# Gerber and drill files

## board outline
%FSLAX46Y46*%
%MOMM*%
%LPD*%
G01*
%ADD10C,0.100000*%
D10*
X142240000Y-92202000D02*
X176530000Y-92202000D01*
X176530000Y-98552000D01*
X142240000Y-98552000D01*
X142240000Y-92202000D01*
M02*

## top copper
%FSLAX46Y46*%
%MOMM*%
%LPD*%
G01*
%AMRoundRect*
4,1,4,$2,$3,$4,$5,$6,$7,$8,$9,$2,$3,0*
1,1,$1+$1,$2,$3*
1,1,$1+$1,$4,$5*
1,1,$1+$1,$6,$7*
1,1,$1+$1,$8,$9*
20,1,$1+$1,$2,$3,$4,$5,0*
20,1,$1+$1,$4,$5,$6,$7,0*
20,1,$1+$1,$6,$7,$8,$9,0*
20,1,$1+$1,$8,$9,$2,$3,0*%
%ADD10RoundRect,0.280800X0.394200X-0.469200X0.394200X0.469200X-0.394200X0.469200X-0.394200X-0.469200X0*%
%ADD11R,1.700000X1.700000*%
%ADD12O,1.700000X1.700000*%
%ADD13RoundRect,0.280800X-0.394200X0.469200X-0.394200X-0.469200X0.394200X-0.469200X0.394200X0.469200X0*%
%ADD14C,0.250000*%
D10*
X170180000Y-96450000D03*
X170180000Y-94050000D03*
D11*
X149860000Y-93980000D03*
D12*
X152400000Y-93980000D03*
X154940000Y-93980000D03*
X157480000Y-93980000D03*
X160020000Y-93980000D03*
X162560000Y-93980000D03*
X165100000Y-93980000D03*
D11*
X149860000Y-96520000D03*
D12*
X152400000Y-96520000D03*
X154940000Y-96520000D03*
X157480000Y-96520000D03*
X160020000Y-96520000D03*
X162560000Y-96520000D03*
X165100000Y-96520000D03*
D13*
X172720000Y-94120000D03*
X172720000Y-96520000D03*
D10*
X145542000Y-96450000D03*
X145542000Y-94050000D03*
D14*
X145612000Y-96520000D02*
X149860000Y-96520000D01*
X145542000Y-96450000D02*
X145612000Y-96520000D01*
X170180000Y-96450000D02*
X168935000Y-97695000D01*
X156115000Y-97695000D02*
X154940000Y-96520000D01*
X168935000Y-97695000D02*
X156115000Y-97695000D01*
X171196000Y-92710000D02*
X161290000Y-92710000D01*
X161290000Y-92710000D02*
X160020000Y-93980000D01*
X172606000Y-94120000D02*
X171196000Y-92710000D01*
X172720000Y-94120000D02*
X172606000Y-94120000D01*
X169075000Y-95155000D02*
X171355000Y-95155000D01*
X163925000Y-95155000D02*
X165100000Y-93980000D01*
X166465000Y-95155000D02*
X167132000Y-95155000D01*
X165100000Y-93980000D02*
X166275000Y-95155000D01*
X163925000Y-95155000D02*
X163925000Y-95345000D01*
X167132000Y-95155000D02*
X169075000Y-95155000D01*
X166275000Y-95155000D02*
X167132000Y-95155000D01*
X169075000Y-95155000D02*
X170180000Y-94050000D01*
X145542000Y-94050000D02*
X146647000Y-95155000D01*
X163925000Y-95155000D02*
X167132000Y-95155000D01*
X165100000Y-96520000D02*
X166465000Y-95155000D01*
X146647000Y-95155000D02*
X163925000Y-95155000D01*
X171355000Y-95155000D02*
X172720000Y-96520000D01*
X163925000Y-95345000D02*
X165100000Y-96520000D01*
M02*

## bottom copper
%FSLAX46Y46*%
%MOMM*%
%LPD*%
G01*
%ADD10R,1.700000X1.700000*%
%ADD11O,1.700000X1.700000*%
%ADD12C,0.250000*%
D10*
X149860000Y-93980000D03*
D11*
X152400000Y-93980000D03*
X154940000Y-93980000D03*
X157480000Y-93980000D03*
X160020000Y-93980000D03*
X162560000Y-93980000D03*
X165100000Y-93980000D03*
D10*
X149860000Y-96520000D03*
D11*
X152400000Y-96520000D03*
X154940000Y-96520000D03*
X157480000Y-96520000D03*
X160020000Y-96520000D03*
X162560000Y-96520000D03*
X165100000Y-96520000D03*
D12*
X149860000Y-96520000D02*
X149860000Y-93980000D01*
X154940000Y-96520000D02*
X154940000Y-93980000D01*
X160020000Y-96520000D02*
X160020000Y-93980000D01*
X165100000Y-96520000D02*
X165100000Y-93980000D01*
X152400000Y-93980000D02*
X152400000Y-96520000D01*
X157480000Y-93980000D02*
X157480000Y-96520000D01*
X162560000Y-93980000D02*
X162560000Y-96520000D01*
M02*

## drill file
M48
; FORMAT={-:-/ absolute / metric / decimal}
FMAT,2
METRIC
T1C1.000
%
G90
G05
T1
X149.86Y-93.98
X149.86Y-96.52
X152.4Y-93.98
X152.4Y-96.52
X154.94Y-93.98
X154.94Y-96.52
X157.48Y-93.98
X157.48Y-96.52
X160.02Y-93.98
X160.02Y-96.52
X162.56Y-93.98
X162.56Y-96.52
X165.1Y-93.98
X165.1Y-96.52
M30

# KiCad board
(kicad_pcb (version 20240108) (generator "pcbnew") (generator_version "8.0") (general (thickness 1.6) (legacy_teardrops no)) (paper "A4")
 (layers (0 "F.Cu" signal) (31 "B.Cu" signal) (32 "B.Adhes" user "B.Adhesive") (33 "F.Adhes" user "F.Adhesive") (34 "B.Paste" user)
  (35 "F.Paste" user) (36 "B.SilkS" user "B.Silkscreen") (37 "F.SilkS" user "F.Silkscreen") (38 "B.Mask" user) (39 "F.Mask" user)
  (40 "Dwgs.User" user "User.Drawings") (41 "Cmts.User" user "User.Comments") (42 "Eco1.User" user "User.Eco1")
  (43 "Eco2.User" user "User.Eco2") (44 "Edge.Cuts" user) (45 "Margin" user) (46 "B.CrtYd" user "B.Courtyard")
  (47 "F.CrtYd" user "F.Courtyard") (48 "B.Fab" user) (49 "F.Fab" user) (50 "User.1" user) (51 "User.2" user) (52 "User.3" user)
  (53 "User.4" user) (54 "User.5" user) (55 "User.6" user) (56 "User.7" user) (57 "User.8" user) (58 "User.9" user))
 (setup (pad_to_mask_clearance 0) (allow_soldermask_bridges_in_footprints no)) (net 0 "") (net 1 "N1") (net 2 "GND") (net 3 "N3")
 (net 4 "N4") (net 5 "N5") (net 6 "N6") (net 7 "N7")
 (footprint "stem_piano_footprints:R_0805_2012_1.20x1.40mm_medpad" (layer "F.Cu") (at 170.18 95.25 90)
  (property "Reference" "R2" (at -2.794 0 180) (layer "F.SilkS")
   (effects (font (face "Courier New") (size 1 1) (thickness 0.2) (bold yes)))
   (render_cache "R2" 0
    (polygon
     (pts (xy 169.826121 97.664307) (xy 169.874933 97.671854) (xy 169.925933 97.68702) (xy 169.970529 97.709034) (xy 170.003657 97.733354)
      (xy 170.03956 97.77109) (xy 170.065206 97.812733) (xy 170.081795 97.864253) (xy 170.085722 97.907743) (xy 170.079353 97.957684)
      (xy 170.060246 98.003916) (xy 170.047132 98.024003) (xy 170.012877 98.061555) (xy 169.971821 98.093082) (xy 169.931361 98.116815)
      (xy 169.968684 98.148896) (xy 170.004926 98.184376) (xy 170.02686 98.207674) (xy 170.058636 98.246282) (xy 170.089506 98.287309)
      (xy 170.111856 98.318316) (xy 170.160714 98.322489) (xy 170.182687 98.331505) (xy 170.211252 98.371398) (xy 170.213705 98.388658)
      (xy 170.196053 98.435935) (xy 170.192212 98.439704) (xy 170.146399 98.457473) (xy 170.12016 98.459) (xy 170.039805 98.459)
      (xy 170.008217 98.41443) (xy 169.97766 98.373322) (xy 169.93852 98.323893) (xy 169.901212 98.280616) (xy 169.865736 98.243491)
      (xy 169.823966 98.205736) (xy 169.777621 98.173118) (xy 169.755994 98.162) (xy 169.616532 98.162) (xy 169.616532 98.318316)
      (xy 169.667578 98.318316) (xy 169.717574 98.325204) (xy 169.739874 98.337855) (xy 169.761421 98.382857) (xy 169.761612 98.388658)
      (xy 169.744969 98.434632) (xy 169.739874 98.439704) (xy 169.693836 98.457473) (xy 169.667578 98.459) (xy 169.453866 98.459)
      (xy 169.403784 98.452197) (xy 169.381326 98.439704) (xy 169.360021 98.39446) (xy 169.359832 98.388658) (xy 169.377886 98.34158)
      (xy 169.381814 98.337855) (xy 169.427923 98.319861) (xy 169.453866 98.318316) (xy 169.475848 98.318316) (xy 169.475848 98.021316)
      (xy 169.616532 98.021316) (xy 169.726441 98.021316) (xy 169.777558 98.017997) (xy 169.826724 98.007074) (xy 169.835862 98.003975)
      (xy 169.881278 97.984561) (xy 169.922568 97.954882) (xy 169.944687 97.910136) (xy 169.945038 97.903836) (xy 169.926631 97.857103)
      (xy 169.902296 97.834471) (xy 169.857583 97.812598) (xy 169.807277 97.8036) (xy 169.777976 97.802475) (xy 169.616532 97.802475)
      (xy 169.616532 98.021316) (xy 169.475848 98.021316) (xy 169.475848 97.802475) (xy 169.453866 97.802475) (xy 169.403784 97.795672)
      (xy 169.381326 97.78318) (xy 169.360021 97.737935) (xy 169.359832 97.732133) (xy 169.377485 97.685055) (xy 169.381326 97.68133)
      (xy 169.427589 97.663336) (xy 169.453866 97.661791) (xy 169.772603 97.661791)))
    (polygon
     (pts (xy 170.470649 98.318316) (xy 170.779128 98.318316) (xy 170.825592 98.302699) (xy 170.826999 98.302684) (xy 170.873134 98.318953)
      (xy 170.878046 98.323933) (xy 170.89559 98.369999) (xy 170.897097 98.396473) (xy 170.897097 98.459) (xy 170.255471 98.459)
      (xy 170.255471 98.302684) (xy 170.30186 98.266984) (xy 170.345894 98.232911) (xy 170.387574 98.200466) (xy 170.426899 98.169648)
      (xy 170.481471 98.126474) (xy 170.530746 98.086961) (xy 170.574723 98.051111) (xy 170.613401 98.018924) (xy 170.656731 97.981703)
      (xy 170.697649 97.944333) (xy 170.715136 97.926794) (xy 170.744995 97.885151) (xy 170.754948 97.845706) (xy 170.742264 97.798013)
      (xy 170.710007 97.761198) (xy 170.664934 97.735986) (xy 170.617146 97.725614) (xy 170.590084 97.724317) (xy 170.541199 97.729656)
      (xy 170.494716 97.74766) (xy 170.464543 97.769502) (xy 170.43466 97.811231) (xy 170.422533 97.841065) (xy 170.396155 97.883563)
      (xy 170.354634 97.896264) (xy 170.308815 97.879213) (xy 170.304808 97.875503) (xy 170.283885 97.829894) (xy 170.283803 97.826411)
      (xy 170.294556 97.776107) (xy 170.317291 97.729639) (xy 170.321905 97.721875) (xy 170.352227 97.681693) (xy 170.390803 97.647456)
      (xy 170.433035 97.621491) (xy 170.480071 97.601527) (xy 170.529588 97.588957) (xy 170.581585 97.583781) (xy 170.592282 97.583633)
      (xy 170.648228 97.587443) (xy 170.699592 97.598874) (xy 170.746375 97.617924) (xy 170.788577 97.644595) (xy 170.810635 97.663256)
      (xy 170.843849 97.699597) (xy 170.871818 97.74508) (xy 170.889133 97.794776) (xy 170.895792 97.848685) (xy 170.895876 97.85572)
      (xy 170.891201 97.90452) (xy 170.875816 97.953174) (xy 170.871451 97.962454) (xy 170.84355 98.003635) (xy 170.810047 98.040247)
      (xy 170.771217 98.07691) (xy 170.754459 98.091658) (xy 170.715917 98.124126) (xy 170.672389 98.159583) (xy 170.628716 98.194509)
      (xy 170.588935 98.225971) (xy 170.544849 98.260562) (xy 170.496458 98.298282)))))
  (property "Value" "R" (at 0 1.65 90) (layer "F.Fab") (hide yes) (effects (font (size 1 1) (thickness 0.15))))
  (pad "1" smd roundrect (at -1.2 0 90) (size 1.5 1.35) (layers "F.Cu" "F.Paste" "F.Mask") (roundrect_rratio 0.208) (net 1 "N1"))
  (pad "2" smd roundrect (at 1.2 0 90) (size 1.5 1.35) (layers "F.Cu" "F.Paste" "F.Mask") (roundrect_rratio 0.208) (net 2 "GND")))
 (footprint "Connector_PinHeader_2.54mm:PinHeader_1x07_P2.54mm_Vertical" (layer "F.Cu") (at 149.86 93.98 90)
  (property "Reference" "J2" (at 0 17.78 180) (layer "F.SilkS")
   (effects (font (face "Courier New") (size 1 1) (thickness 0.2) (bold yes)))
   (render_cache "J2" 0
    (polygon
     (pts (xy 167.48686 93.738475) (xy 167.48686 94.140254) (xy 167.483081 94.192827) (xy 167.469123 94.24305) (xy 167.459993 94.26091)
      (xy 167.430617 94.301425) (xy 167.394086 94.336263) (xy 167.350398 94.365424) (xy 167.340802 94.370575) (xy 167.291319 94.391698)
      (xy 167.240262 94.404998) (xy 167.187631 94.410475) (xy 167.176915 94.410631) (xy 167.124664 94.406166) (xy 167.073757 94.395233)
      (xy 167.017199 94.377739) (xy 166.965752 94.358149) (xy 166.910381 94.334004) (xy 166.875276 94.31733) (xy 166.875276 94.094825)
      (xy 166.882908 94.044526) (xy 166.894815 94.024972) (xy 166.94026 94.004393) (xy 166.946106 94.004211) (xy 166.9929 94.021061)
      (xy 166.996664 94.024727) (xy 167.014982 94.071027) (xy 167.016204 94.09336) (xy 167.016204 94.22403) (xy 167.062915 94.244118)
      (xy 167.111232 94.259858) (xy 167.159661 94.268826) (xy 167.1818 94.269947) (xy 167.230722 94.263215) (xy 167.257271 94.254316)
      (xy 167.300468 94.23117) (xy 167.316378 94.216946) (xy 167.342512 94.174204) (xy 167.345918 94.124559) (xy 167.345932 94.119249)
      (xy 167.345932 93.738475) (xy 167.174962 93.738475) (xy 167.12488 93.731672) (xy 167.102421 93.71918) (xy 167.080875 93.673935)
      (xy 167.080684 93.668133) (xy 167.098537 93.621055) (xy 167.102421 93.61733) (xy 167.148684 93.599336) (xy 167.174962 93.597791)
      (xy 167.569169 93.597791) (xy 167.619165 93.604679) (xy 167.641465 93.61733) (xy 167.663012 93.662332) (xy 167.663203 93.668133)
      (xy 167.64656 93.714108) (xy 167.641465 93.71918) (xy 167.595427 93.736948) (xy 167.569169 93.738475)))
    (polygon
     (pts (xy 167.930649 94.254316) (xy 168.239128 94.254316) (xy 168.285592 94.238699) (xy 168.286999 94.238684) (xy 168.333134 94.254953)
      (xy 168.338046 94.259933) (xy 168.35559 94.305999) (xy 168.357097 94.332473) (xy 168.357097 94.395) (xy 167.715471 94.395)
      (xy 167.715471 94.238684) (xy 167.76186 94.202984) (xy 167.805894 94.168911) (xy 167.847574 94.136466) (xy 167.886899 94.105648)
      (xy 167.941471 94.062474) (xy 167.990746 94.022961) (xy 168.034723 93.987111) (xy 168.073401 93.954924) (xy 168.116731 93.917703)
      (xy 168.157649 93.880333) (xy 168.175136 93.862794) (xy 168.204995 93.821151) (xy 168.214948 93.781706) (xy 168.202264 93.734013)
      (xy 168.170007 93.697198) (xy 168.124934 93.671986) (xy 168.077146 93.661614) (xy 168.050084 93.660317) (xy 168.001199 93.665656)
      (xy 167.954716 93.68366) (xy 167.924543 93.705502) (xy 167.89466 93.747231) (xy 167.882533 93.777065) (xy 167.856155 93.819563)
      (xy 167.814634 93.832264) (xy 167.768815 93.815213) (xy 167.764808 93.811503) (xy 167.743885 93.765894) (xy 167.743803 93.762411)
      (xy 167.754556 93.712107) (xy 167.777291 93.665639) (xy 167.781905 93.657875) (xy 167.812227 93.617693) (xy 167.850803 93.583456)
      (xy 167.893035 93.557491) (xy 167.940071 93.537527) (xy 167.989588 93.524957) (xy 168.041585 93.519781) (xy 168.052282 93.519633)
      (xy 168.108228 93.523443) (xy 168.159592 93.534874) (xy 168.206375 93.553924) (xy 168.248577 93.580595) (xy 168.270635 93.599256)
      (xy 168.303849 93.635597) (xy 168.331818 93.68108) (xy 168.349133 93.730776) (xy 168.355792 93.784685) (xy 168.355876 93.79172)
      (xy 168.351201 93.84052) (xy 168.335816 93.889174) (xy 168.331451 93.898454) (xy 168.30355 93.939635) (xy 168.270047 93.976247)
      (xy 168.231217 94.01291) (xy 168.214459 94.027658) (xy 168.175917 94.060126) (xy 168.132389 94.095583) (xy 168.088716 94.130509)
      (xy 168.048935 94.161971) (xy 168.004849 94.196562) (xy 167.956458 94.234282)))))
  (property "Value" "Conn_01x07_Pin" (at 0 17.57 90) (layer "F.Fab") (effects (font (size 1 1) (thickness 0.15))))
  (pad "1" thru_hole rect (at 0 0 90) (size 1.7 1.7) (drill 1) (layers "*.Cu" "*.Mask") (remove_unused_layers no) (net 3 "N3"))
  (pad "2" thru_hole oval (at 0 2.54 90) (size 1.7 1.7) (drill 1) (layers "*.Cu" "*.Mask") (remove_unused_layers no) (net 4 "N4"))
  (pad "3" thru_hole oval (at 0 5.08 90) (size 1.7 1.7) (drill 1) (layers "*.Cu" "*.Mask") (remove_unused_layers no) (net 1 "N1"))
  (pad "4" thru_hole oval (at 0 7.62 90) (size 1.7 1.7) (drill 1) (layers "*.Cu" "*.Mask") (remove_unused_layers no) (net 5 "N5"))
  (pad "5" thru_hole oval (at 0 10.16 90) (size 1.7 1.7) (drill 1) (layers "*.Cu" "*.Mask") (remove_unused_layers no) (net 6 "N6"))
  (pad "6" thru_hole oval (at 0 12.7 90) (size 1.7 1.7) (drill 1) (layers "*.Cu" "*.Mask") (remove_unused_layers no) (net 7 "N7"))
  (pad "7" thru_hole oval (at 0 15.24 90) (size 1.7 1.7) (drill 1) (layers "*.Cu" "*.Mask") (remove_unused_layers no) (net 2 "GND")))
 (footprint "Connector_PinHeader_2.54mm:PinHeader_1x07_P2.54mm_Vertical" (layer "F.Cu") (at 149.86 96.52 90)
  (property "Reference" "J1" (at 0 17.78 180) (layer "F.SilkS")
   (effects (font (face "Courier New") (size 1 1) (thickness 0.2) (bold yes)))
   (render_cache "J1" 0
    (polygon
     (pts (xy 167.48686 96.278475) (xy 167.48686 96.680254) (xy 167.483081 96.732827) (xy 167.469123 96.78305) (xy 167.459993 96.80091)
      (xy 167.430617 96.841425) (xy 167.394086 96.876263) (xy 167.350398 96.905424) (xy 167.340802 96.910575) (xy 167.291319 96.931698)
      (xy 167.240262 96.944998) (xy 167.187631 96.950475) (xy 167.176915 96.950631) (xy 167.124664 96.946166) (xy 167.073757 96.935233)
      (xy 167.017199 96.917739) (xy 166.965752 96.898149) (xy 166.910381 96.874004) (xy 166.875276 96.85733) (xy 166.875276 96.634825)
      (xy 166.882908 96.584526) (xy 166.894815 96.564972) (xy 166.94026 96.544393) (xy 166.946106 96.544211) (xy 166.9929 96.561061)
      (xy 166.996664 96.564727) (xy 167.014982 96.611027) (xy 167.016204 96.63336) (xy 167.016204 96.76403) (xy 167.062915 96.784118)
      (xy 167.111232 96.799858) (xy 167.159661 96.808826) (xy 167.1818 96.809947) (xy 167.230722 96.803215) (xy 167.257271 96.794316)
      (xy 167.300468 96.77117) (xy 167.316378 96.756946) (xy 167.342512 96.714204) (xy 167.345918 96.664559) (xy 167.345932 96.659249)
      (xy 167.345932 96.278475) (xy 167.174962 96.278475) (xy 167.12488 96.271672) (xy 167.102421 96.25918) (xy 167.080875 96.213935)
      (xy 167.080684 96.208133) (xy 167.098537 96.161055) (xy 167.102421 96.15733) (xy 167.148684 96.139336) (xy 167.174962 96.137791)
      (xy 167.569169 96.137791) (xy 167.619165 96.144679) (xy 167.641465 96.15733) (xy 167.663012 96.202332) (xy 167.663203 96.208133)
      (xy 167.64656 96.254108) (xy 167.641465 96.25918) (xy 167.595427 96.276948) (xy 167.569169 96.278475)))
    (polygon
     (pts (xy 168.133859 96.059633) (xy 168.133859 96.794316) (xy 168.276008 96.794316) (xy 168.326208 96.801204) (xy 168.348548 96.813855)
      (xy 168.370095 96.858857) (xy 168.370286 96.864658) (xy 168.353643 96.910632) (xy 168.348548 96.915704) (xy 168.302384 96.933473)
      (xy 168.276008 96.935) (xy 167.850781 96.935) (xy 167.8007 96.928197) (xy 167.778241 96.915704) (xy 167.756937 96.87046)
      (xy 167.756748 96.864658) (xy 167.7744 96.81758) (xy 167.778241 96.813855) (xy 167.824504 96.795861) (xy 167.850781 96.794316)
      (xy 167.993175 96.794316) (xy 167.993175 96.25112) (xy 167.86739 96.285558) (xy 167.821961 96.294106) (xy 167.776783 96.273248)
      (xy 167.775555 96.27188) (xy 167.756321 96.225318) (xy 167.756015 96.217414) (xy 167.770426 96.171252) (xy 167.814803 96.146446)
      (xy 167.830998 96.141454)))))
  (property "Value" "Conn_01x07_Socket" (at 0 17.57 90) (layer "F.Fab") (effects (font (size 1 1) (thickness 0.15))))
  (pad "1" thru_hole rect (at 0 0 90) (size 1.7 1.7) (drill 1) (layers "*.Cu" "*.Mask") (remove_unused_layers no) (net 3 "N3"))
  (pad "2" thru_hole oval (at 0 2.54 90) (size 1.7 1.7) (drill 1) (layers "*.Cu" "*.Mask") (remove_unused_layers no) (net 4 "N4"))
  (pad "3" thru_hole oval (at 0 5.08 90) (size 1.7 1.7) (drill 1) (layers "*.Cu" "*.Mask") (remove_unused_layers no) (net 1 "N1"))
  (pad "4" thru_hole oval (at 0 7.62 90) (size 1.7 1.7) (drill 1) (layers "*.Cu" "*.Mask") (remove_unused_layers no) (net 5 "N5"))
  (pad "5" thru_hole oval (at 0 10.16 90) (size 1.7 1.7) (drill 1) (layers "*.Cu" "*.Mask") (remove_unused_layers no) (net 6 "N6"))
  (pad "6" thru_hole oval (at 0 12.7 90) (size 1.7 1.7) (drill 1) (layers "*.Cu" "*.Mask") (remove_unused_layers no) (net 7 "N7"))
  (pad "7" thru_hole oval (at 0 15.24 90) (size 1.7 1.7) (drill 1) (layers "*.Cu" "*.Mask") (remove_unused_layers no) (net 2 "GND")))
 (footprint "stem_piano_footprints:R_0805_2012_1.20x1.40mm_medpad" (layer "F.Cu") (at 172.72 95.32 -90)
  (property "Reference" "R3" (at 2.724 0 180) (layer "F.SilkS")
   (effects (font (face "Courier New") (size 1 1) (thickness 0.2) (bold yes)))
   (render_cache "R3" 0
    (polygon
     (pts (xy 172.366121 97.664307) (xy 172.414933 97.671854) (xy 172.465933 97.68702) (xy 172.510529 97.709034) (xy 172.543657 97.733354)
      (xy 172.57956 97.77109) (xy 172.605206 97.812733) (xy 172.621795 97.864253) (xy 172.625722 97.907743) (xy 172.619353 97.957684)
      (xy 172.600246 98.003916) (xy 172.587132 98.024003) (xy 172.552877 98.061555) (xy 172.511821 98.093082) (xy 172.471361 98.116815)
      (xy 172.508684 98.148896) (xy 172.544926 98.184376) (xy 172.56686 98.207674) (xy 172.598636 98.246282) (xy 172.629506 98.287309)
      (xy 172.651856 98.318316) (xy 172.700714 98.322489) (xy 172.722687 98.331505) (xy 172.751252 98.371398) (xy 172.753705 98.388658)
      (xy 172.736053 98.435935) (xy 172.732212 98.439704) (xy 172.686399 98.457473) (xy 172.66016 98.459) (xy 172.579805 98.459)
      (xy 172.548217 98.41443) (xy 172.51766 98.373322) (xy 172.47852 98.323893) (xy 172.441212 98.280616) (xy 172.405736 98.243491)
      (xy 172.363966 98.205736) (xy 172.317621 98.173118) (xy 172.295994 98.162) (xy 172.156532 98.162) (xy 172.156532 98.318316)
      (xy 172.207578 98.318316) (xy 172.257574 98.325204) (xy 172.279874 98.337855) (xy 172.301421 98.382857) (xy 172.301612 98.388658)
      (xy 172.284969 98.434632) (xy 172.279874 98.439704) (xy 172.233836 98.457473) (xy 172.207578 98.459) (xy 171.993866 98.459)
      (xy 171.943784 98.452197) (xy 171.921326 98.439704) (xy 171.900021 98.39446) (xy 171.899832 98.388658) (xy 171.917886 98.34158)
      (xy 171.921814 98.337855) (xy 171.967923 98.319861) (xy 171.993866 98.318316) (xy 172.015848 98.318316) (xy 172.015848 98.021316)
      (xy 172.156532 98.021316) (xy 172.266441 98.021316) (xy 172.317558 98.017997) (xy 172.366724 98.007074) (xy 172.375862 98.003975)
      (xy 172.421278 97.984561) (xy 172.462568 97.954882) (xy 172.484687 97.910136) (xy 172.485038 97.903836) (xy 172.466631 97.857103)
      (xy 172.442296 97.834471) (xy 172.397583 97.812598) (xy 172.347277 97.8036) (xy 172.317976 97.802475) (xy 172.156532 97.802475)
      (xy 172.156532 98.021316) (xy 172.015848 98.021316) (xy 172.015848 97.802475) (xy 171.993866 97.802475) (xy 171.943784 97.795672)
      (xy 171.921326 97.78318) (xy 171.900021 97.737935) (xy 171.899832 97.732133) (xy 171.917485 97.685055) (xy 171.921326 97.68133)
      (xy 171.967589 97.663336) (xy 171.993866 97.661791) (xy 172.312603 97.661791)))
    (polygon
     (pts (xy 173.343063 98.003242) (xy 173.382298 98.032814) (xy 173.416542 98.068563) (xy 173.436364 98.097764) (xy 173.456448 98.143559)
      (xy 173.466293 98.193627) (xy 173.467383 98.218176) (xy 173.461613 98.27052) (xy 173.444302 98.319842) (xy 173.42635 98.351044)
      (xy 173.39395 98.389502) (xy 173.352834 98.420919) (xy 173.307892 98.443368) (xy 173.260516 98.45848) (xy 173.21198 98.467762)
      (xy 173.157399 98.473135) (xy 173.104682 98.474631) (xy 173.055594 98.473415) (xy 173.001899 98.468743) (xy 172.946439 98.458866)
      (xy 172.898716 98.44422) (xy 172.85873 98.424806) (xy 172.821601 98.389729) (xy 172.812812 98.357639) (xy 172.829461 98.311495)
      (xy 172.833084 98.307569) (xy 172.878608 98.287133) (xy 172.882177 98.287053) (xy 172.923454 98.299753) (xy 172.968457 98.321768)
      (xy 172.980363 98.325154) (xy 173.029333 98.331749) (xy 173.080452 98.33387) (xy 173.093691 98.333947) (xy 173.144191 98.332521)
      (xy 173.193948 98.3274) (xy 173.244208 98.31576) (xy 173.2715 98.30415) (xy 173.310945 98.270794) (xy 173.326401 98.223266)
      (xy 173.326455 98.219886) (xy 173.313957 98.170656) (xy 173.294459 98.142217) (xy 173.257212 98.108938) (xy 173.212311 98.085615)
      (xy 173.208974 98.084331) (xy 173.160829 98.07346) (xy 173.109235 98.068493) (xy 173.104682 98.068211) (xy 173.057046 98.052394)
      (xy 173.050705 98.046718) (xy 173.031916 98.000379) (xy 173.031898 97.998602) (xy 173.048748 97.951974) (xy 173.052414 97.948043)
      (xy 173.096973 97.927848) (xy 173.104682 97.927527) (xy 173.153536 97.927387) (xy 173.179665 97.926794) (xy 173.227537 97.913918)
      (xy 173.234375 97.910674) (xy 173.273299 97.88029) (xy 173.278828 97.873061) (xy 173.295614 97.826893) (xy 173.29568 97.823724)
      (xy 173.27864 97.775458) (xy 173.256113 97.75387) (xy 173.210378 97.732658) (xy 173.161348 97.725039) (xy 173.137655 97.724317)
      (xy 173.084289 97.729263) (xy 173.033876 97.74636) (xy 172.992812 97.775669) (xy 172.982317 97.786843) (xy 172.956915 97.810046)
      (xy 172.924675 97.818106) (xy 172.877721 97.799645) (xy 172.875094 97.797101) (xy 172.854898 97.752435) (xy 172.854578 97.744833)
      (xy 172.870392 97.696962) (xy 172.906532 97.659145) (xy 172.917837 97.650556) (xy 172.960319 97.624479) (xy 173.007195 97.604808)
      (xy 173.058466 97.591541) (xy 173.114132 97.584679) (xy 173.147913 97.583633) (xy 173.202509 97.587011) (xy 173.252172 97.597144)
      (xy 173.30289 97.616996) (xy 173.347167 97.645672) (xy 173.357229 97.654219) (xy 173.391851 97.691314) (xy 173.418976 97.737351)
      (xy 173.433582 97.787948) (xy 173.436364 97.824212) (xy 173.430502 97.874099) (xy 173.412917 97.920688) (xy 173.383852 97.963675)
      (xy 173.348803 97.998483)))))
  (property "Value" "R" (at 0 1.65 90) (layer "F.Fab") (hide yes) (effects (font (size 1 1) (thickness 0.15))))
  (pad "1" smd roundrect (at -1.2 0 270) (size 1.5 1.35) (layers "F.Cu" "F.Paste" "F.Mask") (roundrect_rratio 0.208) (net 6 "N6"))
  (pad "2" smd roundrect (at 1.2 0 270) (size 1.5 1.35) (layers "F.Cu" "F.Paste" "F.Mask") (roundrect_rratio 0.208) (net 2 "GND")))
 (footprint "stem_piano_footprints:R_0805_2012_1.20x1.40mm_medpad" (layer "F.Cu") (at 145.542 95.25 90)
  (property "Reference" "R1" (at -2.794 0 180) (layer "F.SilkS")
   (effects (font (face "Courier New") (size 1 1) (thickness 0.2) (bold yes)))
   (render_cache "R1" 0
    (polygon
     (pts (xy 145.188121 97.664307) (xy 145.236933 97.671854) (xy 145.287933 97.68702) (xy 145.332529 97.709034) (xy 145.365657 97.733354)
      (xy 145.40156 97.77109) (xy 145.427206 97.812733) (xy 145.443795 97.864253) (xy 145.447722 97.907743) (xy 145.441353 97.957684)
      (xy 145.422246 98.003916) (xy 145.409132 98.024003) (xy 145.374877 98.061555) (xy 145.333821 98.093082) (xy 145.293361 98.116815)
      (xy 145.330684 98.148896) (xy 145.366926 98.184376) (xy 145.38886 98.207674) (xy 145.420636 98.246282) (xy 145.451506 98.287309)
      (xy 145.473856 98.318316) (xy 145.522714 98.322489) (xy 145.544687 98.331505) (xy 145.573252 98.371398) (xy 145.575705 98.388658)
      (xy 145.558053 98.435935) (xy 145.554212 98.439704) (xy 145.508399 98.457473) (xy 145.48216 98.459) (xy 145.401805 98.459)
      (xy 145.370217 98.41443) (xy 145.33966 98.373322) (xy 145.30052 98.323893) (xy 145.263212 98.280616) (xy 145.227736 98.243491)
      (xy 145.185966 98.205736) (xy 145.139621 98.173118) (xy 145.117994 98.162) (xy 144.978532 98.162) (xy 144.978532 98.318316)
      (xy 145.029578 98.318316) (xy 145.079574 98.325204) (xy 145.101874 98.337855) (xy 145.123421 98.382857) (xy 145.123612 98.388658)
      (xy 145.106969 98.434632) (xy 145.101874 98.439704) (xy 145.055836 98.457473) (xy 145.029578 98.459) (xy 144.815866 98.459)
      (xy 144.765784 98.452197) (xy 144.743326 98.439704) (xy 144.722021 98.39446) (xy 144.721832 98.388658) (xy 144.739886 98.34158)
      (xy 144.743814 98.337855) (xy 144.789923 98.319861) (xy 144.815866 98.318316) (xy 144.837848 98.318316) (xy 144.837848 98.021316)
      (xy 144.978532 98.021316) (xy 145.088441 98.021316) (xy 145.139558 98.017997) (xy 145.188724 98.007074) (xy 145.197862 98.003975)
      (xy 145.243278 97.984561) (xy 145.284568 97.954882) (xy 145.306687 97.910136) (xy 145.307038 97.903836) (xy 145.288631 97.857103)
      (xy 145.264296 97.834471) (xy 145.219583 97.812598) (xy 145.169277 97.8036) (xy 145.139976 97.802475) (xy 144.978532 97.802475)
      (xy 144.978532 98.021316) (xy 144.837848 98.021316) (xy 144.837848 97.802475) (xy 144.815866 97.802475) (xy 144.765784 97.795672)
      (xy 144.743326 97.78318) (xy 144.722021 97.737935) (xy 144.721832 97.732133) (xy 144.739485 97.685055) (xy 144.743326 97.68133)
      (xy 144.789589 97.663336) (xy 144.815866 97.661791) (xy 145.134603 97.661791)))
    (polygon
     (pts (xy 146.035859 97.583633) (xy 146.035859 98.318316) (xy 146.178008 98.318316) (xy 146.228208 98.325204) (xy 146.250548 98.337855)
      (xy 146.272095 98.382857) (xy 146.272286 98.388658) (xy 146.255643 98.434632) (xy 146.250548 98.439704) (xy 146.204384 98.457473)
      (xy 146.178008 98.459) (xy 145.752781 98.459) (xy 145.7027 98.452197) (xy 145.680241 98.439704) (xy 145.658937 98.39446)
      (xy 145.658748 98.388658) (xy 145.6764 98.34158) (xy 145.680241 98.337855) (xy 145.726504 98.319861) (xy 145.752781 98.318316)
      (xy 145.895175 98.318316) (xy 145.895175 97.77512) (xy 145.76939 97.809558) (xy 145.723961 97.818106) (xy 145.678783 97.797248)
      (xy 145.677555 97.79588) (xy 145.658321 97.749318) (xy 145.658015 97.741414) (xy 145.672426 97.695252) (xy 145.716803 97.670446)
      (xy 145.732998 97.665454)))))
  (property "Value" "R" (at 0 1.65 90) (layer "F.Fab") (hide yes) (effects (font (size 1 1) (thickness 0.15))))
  (pad "1" smd roundrect (at -1.2 0 90) (size 1.5 1.35) (layers "F.Cu" "F.Paste" "F.Mask") (roundrect_rratio 0.208) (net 3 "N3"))
  (pad "2" smd roundrect (at 1.2 0 90) (size 1.5 1.35) (layers "F.Cu" "F.Paste" "F.Mask") (roundrect_rratio 0.208) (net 2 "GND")))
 (gr_rect (start 142.24 92.202) (end 176.53 98.552) (stroke (width 0.1) (type default)) (fill none) (layer "Edge.Cuts"))
 (segment (start 145.612 96.52) (end 149.86 96.52) (width 0.25) (layer "F.Cu") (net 3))
 (segment (start 145.542 96.45) (end 145.612 96.52) (width 0.25) (layer "F.Cu") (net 3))
 (segment (start 149.86 96.52) (end 149.86 93.98) (width 0.25) (layer "B.Cu") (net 3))
 (segment (start 170.18 96.45) (end 168.935 97.695) (width 0.25) (layer "F.Cu") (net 1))
 (segment (start 156.115 97.695) (end 154.94 96.52) (width 0.25) (layer "F.Cu") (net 1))
 (segment (start 168.935 97.695) (end 156.115 97.695) (width 0.25) (layer "F.Cu") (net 1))
 (segment (start 154.94 96.52) (end 154.94 93.98) (width 0.25) (layer "B.Cu") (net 1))
 (segment (start 171.196 92.71) (end 161.29 92.71) (width 0.25) (layer "F.Cu") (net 6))
 (segment (start 161.29 92.71) (end 160.02 93.98) (width 0.25) (layer "F.Cu") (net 6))
 (segment (start 172.606 94.12) (end 171.196 92.71) (width 0.25) (layer "F.Cu") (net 6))
 (segment (start 172.72 94.12) (end 172.606 94.12) (width 0.25) (layer "F.Cu") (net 6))
 (segment (start 160.02 96.52) (end 160.02 93.98) (width 0.25) (layer "B.Cu") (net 6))
 (segment (start 169.075 95.155) (end 171.355 95.155) (width 0.25) (layer "F.Cu") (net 2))
 (segment (start 163.925 95.155) (end 165.1 93.98) (width 0.25) (layer "F.Cu") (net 2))
 (segment (start 166.465 95.155) (end 167.132 95.155) (width 0.25) (layer "F.Cu") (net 2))
 (segment (start 165.1 93.98) (end 166.275 95.155) (width 0.25) (layer "F.Cu") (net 2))
 (segment (start 163.925 95.155) (end 163.925 95.345) (width 0.25) (layer "F.Cu") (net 2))
 (segment (start 167.132 95.155) (end 169.075 95.155) (width 0.25) (layer "F.Cu") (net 2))
 (segment (start 166.275 95.155) (end 167.132 95.155) (width 0.25) (layer "F.Cu") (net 2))
 (segment (start 169.075 95.155) (end 170.18 94.05) (width 0.25) (layer "F.Cu") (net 2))
 (segment (start 145.542 94.05) (end 146.647 95.155) (width 0.25) (layer "F.Cu") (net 2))
 (segment (start 163.925 95.155) (end 167.132 95.155) (width 0.25) (layer "F.Cu") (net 2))
 (segment (start 165.1 96.52) (end 166.465 95.155) (width 0.25) (layer "F.Cu") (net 2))
 (segment (start 146.647 95.155) (end 163.925 95.155) (width 0.25) (layer "F.Cu") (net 2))
 (segment (start 171.355 95.155) (end 172.72 96.52) (width 0.25) (layer "F.Cu") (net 2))
 (segment (start 163.925 95.345) (end 165.1 96.52) (width 0.25) (layer "F.Cu") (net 2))
 (segment (start 165.1 96.52) (end 165.1 93.98) (width 0.25) (layer "B.Cu") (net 2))
 (segment (start 152.4 93.98) (end 152.4 96.52) (width 0.25) (layer "B.Cu") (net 4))
 (segment (start 157.48 93.98) (end 157.48 96.52) (width 0.25) (layer "B.Cu") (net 5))
 (segment (start 162.56 93.98) (end 162.56 96.52) (width 0.25) (layer "B.Cu") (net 7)))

